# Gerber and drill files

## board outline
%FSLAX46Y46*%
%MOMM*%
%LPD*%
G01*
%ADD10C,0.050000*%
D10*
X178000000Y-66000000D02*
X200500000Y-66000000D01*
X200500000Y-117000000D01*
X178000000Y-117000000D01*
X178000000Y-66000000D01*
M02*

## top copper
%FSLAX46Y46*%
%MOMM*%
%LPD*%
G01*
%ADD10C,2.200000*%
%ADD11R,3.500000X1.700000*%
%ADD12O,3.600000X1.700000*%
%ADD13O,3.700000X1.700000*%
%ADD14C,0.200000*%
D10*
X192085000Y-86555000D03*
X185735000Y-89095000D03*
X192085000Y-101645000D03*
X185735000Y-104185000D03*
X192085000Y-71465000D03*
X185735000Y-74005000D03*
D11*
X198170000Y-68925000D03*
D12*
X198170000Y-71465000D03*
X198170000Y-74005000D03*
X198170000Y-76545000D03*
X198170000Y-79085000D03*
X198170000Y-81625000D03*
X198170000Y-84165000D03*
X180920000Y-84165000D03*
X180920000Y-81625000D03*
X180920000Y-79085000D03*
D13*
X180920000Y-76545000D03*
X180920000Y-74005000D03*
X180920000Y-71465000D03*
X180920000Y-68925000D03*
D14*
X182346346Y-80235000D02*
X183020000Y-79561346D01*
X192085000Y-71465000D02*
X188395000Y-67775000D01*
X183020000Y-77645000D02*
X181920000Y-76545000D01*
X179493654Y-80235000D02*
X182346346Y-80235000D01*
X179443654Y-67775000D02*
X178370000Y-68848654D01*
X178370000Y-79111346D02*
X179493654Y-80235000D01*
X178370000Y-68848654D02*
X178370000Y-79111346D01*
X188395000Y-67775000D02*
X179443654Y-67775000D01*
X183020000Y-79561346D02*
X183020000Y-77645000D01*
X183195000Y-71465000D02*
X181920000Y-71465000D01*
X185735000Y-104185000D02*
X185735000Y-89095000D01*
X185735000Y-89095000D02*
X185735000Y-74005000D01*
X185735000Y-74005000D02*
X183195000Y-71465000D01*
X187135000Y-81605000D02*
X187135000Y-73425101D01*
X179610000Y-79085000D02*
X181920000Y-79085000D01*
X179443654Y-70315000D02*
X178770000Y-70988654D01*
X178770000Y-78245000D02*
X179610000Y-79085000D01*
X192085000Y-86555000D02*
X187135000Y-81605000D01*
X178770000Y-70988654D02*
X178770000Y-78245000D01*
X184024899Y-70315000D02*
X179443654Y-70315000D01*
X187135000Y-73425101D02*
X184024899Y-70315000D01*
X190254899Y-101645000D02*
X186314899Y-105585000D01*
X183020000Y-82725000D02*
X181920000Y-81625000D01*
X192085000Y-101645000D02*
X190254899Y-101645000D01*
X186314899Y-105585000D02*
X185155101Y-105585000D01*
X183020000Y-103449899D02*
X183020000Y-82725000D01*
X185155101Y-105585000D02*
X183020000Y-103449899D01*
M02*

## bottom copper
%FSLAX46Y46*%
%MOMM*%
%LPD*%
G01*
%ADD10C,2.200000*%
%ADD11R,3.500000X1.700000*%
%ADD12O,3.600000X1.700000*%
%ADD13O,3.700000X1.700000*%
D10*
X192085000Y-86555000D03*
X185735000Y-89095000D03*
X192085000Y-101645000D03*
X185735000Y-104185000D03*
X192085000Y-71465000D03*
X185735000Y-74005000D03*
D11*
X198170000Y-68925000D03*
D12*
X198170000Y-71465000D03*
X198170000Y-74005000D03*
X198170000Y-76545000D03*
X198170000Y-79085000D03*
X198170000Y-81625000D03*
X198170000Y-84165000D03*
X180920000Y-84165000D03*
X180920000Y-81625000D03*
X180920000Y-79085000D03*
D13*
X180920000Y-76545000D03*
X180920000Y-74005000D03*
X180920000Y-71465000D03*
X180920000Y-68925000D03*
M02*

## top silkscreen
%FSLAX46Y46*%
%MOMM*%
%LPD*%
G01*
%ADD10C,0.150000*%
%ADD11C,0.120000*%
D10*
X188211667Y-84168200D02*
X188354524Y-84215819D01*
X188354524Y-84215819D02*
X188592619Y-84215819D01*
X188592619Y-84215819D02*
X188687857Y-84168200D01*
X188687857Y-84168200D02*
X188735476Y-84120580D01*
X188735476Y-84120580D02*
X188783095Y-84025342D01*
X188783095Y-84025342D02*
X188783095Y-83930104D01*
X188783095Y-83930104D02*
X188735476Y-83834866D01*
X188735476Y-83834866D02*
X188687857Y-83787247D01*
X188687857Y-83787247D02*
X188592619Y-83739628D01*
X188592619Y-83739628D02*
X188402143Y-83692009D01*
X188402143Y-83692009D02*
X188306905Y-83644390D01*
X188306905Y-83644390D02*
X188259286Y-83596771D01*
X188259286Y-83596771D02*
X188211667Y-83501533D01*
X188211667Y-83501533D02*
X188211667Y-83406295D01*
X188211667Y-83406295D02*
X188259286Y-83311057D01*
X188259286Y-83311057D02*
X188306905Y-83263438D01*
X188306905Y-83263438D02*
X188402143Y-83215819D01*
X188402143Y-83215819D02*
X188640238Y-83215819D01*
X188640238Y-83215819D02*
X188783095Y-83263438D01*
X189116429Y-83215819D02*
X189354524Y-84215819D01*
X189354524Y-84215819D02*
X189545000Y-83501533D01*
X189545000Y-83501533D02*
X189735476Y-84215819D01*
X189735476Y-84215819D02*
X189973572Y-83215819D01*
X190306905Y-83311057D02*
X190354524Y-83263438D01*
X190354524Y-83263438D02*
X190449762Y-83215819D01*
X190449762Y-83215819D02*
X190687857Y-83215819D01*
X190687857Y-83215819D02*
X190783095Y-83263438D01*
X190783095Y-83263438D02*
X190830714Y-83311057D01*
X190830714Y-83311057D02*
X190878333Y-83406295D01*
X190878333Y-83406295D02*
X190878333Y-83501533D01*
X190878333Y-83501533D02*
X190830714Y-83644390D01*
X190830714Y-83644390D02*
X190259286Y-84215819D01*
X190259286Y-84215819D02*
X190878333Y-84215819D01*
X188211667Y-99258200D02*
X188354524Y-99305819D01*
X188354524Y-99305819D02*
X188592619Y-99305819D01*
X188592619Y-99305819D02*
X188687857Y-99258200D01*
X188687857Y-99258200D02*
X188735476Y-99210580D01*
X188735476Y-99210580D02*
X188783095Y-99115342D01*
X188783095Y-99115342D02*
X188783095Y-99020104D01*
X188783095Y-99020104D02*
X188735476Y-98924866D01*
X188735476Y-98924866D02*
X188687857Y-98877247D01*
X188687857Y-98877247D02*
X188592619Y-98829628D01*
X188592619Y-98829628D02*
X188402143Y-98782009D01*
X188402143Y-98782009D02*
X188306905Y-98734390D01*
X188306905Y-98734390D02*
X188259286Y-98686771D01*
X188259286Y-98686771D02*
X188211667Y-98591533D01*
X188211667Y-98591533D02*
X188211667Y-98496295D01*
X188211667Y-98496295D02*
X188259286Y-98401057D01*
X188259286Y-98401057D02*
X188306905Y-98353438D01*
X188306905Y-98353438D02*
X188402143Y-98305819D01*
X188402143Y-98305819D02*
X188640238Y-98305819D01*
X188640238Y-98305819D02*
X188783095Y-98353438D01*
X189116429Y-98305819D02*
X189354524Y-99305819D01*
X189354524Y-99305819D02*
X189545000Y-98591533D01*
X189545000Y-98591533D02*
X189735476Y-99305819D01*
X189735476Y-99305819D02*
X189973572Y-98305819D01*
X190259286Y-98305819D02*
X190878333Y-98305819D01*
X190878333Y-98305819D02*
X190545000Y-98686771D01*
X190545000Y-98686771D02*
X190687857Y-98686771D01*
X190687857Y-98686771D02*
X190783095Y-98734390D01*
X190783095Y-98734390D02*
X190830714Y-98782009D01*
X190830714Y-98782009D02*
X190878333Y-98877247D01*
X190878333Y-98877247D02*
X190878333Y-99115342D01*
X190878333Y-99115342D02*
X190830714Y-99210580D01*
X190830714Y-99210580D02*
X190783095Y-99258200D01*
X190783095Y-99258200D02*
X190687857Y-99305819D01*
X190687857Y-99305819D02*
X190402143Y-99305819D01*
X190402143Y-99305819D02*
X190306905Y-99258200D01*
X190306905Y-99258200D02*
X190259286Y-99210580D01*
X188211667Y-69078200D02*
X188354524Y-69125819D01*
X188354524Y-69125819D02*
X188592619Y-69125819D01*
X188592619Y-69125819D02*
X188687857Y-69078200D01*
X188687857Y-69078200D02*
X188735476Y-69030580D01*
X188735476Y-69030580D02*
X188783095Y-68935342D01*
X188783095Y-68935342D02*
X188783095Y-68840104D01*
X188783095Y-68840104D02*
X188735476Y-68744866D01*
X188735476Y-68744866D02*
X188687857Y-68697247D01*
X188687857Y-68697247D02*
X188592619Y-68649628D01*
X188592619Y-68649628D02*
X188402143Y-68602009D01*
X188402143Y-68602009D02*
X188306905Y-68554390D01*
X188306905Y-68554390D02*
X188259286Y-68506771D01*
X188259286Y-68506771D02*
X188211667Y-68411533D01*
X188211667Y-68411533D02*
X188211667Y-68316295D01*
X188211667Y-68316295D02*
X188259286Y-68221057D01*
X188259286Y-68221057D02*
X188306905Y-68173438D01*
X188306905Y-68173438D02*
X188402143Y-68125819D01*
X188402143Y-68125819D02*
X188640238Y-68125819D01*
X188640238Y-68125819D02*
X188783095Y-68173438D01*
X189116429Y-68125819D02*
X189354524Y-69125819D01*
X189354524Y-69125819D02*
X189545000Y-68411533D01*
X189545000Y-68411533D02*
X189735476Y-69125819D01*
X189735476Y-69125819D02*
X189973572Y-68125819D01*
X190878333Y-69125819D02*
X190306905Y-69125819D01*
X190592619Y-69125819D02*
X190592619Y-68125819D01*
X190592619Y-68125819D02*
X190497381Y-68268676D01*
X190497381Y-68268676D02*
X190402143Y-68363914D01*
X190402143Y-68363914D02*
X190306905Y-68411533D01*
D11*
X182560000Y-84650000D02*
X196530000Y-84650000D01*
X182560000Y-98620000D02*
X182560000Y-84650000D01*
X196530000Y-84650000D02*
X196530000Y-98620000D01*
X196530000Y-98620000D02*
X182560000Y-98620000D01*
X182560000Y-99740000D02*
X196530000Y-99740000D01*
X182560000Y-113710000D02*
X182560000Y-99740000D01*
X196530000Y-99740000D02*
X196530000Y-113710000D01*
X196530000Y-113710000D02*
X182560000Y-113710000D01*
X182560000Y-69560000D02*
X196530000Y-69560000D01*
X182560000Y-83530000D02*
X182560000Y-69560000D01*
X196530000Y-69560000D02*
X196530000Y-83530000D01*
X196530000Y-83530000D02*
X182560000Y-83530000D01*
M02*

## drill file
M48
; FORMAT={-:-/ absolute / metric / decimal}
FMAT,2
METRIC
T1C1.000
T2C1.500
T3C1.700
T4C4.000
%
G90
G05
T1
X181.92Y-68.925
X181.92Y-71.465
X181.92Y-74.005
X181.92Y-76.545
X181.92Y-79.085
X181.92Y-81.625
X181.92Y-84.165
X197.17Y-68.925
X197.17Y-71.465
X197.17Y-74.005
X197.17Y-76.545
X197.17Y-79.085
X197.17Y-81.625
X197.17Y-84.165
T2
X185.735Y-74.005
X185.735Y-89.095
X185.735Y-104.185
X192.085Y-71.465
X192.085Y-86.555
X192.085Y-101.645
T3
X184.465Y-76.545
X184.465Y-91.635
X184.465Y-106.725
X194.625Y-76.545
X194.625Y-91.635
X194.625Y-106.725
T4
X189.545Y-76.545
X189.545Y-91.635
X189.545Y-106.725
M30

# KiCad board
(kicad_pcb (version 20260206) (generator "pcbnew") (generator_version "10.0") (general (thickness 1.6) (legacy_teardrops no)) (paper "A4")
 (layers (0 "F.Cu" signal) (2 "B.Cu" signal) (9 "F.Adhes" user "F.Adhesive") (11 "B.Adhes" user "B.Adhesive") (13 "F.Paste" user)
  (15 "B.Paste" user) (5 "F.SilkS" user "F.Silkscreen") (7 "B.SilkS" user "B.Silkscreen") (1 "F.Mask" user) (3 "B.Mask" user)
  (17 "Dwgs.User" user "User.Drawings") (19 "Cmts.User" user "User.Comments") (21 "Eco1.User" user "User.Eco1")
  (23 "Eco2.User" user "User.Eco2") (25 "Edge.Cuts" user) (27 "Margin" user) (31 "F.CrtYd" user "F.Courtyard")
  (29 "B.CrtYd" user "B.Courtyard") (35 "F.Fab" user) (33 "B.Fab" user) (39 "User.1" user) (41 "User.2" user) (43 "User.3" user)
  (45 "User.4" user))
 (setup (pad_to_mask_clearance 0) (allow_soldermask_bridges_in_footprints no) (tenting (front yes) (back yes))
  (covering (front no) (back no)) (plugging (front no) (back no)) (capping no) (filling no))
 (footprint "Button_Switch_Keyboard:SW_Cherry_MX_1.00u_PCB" (layer "F.Cu") (at 192.085 86.555)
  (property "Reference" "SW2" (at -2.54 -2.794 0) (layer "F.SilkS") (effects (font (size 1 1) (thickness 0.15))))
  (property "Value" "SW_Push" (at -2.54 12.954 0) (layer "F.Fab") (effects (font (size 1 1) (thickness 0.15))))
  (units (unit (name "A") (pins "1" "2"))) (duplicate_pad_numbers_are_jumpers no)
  (fp_line (start -9.525 -1.905) (end 4.445 -1.905) (stroke (width 0.12) (type solid)) (layer "F.SilkS"))
  (fp_line (start -9.525 12.065) (end -9.525 -1.905) (stroke (width 0.12) (type solid)) (layer "F.SilkS"))
  (fp_line (start 4.445 -1.905) (end 4.445 12.065) (stroke (width 0.12) (type solid)) (layer "F.SilkS"))
  (fp_line (start 4.445 12.065) (end -9.525 12.065) (stroke (width 0.12) (type solid)) (layer "F.SilkS"))
  (pad "" np_thru_hole circle (at -7.62 5.08) (size 1.7 1.7) (drill 1.7) (layers "*.Cu" "*.Mask"))
  (pad "" np_thru_hole circle (at -2.54 5.08) (size 4 4) (drill 4) (layers "*.Cu" "*.Mask"))
  (pad "" np_thru_hole circle (at 2.54 5.08) (size 1.7 1.7) (drill 1.7) (layers "*.Cu" "*.Mask"))
  (pad "1" thru_hole circle (at 0 0) (size 2.2 2.2) (drill 1.5) (layers "*.Cu" "*.Mask") (remove_unused_layers no)
   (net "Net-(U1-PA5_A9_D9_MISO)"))
  (pad "2" thru_hole circle (at -6.35 2.54) (size 2.2 2.2) (drill 1.5) (layers "*.Cu" "*.Mask") (remove_unused_layers no) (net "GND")))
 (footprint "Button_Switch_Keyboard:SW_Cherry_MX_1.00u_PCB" (layer "F.Cu") (at 192.085 101.645)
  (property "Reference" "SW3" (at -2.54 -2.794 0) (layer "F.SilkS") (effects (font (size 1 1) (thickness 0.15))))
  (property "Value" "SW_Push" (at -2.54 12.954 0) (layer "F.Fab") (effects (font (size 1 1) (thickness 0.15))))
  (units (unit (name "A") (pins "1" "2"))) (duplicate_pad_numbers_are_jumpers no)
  (fp_line (start -9.525 -1.905) (end 4.445 -1.905) (stroke (width 0.12) (type solid)) (layer "F.SilkS"))
  (fp_line (start -9.525 12.065) (end -9.525 -1.905) (stroke (width 0.12) (type solid)) (layer "F.SilkS"))
  (fp_line (start 4.445 -1.905) (end 4.445 12.065) (stroke (width 0.12) (type solid)) (layer "F.SilkS"))
  (fp_line (start 4.445 12.065) (end -9.525 12.065) (stroke (width 0.12) (type solid)) (layer "F.SilkS"))
  (pad "" np_thru_hole circle (at -7.62 5.08) (size 1.7 1.7) (drill 1.7) (layers "*.Cu" "*.Mask"))
  (pad "" np_thru_hole circle (at -2.54 5.08) (size 4 4) (drill 4) (layers "*.Cu" "*.Mask"))
  (pad "" np_thru_hole circle (at 2.54 5.08) (size 1.7 1.7) (drill 1.7) (layers "*.Cu" "*.Mask"))
  (pad "1" thru_hole circle (at 0 0) (size 2.2 2.2) (drill 1.5) (layers "*.Cu" "*.Mask") (remove_unused_layers no)
   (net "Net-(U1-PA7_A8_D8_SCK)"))
  (pad "2" thru_hole circle (at -6.35 2.54) (size 2.2 2.2) (drill 1.5) (layers "*.Cu" "*.Mask") (remove_unused_layers no) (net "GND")))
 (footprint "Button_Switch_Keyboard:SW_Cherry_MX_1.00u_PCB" (layer "F.Cu") (at 192.085 71.465)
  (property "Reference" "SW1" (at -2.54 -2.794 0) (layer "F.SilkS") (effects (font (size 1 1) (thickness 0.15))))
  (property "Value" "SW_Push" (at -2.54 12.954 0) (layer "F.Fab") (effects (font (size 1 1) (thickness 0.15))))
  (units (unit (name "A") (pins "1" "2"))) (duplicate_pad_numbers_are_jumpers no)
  (fp_line (start -9.525 -1.905) (end 4.445 -1.905) (stroke (width 0.12) (type solid)) (layer "F.SilkS"))
  (fp_line (start -9.525 12.065) (end -9.525 -1.905) (stroke (width 0.12) (type solid)) (layer "F.SilkS"))
  (fp_line (start 4.445 -1.905) (end 4.445 12.065) (stroke (width 0.12) (type solid)) (layer "F.SilkS"))
  (fp_line (start 4.445 12.065) (end -9.525 12.065) (stroke (width 0.12) (type solid)) (layer "F.SilkS"))
  (pad "" np_thru_hole circle (at -7.62 5.08) (size 1.7 1.7) (drill 1.7) (layers "*.Cu" "*.Mask"))
  (pad "" np_thru_hole circle (at -2.54 5.08) (size 4 4) (drill 4) (layers "*.Cu" "*.Mask"))
  (pad "" np_thru_hole circle (at 2.54 5.08) (size 1.7 1.7) (drill 1.7) (layers "*.Cu" "*.Mask"))
  (pad "1" thru_hole circle (at 0 0) (size 2.2 2.2) (drill 1.5) (layers "*.Cu" "*.Mask") (remove_unused_layers no)
   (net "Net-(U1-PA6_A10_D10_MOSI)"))
  (pad "2" thru_hole circle (at -6.35 2.54) (size 2.2 2.2) (drill 1.5) (layers "*.Cu" "*.Mask") (remove_unused_layers no) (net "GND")))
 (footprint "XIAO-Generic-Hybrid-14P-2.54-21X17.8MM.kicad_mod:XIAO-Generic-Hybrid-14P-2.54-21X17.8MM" (layer "B.Cu") (at 189.545 76.545 180)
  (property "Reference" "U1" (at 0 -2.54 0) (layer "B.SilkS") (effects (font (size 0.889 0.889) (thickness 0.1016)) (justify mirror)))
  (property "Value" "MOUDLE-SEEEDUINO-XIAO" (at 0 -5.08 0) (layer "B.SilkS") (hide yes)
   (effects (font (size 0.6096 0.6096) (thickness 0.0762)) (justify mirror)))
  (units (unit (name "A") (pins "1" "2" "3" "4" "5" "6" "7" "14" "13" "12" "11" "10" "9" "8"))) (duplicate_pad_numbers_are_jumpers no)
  (pad "1" thru_hole rect (at -7.625 7.62 180) (size 3.5 1.7) (drill 1 (offset -1 0)) (layers "*.Cu" "*.Mask") (remove_unused_layers no)
   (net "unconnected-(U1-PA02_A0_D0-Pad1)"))
  (pad "2" thru_hole oval (at -7.625 5.08 180) (size 3.6 1.7) (drill 1 (offset -1 0)) (layers "*.Cu" "*.Mask") (remove_unused_layers no)
   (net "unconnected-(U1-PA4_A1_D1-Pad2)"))
  (pad "3" thru_hole oval (at -7.625 2.54 180) (size 3.6 1.7) (drill 1 (offset -1 0)) (layers "*.Cu" "*.Mask") (remove_unused_layers no)
   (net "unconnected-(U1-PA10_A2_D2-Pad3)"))
  (pad "4" thru_hole oval (at -7.625 0 180) (size 3.6 1.7) (drill 1 (offset -1 0)) (layers "*.Cu" "*.Mask") (remove_unused_layers no)
   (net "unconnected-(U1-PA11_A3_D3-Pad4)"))
  (pad "5" thru_hole oval (at -7.625 -2.54 180) (size 3.6 1.7) (drill 1 (offset -1 0)) (layers "*.Cu" "*.Mask") (remove_unused_layers no)
   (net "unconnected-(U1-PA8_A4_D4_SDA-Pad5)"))
  (pad "6" thru_hole oval (at -7.625 -5.08) (size 3.6 1.7) (drill 1 (offset 1 0)) (layers "*.Cu" "*.Mask") (remove_unused_layers no)
   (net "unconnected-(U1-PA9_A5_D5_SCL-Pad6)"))
  (pad "7" thru_hole oval (at -7.625 -7.62 180) (size 3.6 1.7) (drill 1 (offset -1 0)) (layers "*.Cu" "*.Mask") (remove_unused_layers no)
   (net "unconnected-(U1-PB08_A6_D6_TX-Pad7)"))
  (pad "8" thru_hole oval (at 7.625 -7.62 180) (size 3.6 1.7) (drill 1 (offset 1 0)) (layers "*.Cu" "*.Mask") (remove_unused_layers no)
   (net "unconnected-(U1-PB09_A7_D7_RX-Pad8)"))
  (pad "9" thru_hole oval (at 7.625 -5.08 180) (size 3.6 1.7) (drill 1 (offset 1 0)) (layers "*.Cu" "*.Mask") (remove_unused_layers no)
   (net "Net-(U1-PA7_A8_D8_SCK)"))
  (pad "10" thru_hole oval (at 7.625 -2.54 180) (size 3.6 1.7) (drill 1 (offset 1 0)) (layers "*.Cu" "*.Mask") (remove_unused_layers no)
   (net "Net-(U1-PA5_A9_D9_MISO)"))
  (pad "11" thru_hole oval (at 7.625 0 180) (size 3.7 1.7) (drill 1 (offset 1 0)) (layers "*.Cu" "*.Mask") (remove_unused_layers no)
   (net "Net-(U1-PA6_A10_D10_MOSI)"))
  (pad "12" thru_hole oval (at 7.625 2.54 180) (size 3.7 1.7) (drill 1 (offset 1 0)) (layers "*.Cu" "*.Mask") (remove_unused_layers no)
   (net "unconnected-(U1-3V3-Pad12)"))
  (pad "13" thru_hole oval (at 7.625 5.08 180) (size 3.7 1.7) (drill 1 (offset 1 0)) (layers "*.Cu" "*.Mask") (remove_unused_layers no)
   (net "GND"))
  (pad "14" thru_hole oval (at 7.625 7.62 180) (size 3.7 1.7) (drill 1 (offset 1 0)) (layers "*.Cu" "*.Mask") (remove_unused_layers no)
   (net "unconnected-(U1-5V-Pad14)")))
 (gr_rect (start 178 66) (end 200.5 117) (stroke (width 0.05) (type default)) (fill no) (layer "Edge.Cuts"))
 (segment (start 182.346346 80.235) (end 183.02 79.561346) (width 0.2) (layer "F.Cu") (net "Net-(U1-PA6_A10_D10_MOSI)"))
 (segment (start 192.085 71.465) (end 188.395 67.775) (width 0.2) (layer "F.Cu") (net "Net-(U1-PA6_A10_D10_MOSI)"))
 (segment (start 183.02 77.645) (end 181.92 76.545) (width 0.2) (layer "F.Cu") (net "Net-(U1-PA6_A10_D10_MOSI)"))
 (segment (start 179.493654 80.235) (end 182.346346 80.235) (width 0.2) (layer "F.Cu") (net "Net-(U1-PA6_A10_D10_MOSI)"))
 (segment (start 179.443654 67.775) (end 178.37 68.848654) (width 0.2) (layer "F.Cu") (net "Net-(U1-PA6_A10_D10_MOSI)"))
 (segment (start 178.37 79.111346) (end 179.493654 80.235) (width 0.2) (layer "F.Cu") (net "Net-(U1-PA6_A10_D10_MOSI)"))
 (segment (start 178.37 68.848654) (end 178.37 79.111346) (width 0.2) (layer "F.Cu") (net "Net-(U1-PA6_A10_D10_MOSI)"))
 (segment (start 188.395 67.775) (end 179.443654 67.775) (width 0.2) (layer "F.Cu") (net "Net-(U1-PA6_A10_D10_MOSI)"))
 (segment (start 183.02 79.561346) (end 183.02 77.645) (width 0.2) (layer "F.Cu") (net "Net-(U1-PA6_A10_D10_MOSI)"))
 (segment (start 183.195 71.465) (end 181.92 71.465) (width 0.2) (layer "F.Cu") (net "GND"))
 (segment (start 185.735 104.185) (end 185.735 89.095) (width 0.2) (layer "F.Cu") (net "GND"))
 (segment (start 185.735 89.095) (end 185.735 74.005) (width 0.2) (layer "F.Cu") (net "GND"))
 (segment (start 185.735 74.005) (end 183.195 71.465) (width 0.2) (layer "F.Cu") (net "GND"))
 (segment (start 187.135 81.605) (end 187.135 73.425101) (width 0.2) (layer "F.Cu") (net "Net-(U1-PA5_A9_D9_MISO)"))
 (segment (start 179.61 79.085) (end 181.92 79.085) (width 0.2) (layer "F.Cu") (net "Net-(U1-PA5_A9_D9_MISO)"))
 (segment (start 179.443654 70.315) (end 178.77 70.988654) (width 0.2) (layer "F.Cu") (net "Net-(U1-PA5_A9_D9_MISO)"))
 (segment (start 178.77 78.245) (end 179.61 79.085) (width 0.2) (layer "F.Cu") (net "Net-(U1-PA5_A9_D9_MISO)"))
 (segment (start 192.085 86.555) (end 187.135 81.605) (width 0.2) (layer "F.Cu") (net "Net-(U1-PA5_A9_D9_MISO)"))
 (segment (start 178.77 70.988654) (end 178.77 78.245) (width 0.2) (layer "F.Cu") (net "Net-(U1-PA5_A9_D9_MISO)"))
 (segment (start 184.024899 70.315) (end 179.443654 70.315) (width 0.2) (layer "F.Cu") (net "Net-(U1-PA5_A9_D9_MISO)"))
 (segment (start 187.135 73.425101) (end 184.024899 70.315) (width 0.2) (layer "F.Cu") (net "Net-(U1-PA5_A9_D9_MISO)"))
 (segment (start 190.254899 101.645) (end 186.314899 105.585) (width 0.2) (layer "F.Cu") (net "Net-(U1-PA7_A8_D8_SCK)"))
 (segment (start 183.02 82.725) (end 181.92 81.625) (width 0.2) (layer "F.Cu") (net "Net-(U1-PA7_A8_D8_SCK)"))
 (segment (start 192.085 101.645) (end 190.254899 101.645) (width 0.2) (layer "F.Cu") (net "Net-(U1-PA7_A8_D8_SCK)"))
 (segment (start 186.314899 105.585) (end 185.155101 105.585) (width 0.2) (layer "F.Cu") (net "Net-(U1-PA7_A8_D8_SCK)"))
 (segment (start 183.02 103.449899) (end 183.02 82.725) (width 0.2) (layer "F.Cu") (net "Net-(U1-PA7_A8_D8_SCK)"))
 (segment (start 185.155101 105.585) (end 183.02 103.449899) (width 0.2) (layer "F.Cu") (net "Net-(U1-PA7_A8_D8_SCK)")))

